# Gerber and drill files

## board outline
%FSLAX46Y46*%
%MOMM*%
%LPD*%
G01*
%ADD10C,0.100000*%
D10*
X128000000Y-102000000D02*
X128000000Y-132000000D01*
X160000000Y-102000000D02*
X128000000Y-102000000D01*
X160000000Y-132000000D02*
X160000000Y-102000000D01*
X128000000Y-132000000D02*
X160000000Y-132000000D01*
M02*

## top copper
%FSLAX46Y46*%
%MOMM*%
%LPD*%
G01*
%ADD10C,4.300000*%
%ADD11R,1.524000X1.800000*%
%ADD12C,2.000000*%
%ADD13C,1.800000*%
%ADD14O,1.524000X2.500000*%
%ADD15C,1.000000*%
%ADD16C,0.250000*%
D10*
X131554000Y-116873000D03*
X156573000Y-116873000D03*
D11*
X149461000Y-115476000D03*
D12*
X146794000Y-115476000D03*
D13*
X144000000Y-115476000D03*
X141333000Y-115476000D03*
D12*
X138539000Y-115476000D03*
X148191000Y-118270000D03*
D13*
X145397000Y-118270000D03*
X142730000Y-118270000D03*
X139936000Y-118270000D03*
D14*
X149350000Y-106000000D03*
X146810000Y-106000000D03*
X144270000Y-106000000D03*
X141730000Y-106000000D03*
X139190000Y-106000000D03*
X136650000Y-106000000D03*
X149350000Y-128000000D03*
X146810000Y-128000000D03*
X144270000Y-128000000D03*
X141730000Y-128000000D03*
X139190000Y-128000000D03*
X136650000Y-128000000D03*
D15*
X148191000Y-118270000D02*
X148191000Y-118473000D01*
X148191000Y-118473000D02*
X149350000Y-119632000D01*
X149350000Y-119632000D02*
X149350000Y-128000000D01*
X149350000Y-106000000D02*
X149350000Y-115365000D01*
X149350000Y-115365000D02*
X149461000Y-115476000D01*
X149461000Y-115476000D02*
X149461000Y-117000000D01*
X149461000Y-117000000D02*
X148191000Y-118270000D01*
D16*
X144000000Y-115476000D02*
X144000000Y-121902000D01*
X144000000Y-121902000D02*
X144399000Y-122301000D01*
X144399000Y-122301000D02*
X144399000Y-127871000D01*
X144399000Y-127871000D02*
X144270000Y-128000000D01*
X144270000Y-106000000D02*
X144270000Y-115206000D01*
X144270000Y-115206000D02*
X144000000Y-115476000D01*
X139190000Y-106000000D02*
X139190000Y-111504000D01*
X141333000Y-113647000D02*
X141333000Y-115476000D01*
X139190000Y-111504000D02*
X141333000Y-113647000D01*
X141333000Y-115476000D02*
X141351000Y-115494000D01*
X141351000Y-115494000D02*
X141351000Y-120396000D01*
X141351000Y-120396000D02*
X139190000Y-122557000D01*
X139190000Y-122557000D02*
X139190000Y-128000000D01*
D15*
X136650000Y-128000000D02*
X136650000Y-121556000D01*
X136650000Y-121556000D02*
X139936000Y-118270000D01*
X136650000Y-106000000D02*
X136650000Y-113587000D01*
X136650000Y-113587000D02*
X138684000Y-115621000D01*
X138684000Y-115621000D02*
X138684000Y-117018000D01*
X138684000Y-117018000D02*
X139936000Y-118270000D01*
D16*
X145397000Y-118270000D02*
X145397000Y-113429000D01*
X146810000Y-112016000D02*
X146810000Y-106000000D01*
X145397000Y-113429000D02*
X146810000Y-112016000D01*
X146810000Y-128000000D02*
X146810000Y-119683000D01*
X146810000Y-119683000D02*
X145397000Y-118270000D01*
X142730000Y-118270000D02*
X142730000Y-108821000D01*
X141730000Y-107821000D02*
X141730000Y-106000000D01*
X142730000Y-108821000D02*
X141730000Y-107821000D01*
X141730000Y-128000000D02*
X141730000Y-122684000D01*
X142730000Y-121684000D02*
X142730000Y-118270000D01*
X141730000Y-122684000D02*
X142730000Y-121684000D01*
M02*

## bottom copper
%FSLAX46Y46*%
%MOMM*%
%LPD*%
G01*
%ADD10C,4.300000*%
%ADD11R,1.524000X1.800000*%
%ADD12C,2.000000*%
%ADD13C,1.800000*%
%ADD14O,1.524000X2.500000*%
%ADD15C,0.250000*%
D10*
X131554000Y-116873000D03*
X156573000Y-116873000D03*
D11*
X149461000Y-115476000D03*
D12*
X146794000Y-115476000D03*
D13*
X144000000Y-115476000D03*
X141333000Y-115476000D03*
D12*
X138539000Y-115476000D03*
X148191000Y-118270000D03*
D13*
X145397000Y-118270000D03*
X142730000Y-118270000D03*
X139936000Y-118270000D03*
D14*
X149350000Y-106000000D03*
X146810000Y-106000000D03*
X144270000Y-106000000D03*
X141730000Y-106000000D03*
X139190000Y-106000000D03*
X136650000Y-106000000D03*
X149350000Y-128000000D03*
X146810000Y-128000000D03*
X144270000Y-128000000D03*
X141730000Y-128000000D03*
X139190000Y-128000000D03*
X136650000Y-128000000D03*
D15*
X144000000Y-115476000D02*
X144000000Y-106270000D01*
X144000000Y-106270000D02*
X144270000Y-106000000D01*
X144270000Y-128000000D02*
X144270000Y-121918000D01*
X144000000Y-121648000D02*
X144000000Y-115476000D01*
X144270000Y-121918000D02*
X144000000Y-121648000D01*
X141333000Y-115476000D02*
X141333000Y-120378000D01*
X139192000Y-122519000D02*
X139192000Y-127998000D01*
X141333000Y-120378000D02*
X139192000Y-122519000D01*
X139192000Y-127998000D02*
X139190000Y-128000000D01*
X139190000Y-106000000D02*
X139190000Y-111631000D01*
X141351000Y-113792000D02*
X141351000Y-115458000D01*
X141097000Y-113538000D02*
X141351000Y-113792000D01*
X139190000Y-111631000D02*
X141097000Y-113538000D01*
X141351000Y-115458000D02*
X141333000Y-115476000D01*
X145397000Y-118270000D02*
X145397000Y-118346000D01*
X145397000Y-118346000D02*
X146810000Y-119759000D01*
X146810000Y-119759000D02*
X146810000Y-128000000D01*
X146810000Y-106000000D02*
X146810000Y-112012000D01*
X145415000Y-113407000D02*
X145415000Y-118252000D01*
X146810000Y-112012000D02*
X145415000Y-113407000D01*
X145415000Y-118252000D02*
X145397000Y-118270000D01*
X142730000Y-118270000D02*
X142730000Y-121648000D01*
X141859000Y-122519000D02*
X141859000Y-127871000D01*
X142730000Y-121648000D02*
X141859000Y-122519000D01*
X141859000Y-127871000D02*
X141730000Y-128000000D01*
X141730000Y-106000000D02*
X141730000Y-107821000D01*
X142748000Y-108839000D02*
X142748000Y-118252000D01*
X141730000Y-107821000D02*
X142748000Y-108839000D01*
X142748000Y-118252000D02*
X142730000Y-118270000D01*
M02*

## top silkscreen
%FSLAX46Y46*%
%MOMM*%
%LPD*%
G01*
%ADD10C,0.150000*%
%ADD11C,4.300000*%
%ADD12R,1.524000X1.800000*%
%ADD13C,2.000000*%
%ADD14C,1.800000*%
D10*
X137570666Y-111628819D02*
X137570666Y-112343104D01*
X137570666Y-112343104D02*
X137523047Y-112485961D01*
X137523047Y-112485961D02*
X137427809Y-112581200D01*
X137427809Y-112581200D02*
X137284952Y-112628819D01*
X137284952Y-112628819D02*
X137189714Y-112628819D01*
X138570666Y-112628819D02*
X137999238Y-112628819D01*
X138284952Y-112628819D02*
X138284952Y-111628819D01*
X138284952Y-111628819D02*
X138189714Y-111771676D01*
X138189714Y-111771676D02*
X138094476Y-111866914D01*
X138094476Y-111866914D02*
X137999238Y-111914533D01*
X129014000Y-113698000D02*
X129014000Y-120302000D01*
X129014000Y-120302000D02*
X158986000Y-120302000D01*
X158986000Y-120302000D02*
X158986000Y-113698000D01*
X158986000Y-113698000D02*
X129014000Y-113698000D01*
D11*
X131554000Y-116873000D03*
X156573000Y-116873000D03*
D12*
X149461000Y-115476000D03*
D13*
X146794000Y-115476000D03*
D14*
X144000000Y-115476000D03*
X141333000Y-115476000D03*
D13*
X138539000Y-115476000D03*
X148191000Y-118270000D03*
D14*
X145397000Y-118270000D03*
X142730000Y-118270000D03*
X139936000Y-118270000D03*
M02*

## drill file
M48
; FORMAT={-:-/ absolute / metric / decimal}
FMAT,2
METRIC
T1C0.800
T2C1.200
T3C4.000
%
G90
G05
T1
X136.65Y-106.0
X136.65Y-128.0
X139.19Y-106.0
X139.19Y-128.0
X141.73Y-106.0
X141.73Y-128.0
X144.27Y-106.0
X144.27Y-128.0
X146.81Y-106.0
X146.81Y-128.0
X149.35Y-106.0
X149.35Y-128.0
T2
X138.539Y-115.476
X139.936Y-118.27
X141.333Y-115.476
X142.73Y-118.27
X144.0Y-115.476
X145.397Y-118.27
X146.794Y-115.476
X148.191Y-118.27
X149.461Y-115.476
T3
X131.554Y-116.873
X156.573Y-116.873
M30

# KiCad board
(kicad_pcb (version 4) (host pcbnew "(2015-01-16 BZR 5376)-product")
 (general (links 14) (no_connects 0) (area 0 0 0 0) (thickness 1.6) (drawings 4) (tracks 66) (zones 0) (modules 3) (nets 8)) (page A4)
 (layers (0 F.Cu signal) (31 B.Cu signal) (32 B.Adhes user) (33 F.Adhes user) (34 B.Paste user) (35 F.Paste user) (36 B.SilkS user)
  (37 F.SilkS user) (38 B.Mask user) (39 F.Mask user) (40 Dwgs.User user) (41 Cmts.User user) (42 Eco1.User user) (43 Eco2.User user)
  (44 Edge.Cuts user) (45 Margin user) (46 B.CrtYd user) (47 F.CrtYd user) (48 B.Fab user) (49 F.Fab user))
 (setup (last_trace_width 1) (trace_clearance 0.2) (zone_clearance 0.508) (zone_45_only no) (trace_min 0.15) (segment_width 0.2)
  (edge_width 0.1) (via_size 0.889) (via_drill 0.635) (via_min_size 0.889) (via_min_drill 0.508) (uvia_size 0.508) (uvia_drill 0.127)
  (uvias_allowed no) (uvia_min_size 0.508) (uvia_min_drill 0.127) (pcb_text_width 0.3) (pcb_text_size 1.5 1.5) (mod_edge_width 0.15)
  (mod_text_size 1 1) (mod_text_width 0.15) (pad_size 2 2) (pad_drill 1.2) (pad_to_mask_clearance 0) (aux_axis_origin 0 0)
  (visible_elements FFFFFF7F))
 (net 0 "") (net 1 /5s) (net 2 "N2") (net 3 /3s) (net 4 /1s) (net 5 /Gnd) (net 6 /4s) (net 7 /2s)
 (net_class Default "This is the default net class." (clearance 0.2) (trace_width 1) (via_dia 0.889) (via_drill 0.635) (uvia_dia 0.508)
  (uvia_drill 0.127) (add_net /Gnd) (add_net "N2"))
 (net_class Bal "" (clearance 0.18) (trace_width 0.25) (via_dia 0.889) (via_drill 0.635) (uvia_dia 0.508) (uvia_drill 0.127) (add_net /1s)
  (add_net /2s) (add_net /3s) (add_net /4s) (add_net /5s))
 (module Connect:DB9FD (layer F.Cu) (at 144 117)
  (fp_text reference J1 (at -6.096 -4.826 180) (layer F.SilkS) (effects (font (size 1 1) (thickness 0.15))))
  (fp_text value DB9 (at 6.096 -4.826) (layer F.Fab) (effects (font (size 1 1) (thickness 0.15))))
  (fp_line (start -14.986 -3.302) (end -14.986 3.302) (layer F.SilkS) (width 0.15))
  (fp_line (start -14.986 3.302) (end 14.986 3.302) (layer F.SilkS) (width 0.15))
  (fp_line (start 14.986 3.302) (end 14.986 -3.302) (layer F.SilkS) (width 0.15))
  (fp_line (start 14.986 -3.302) (end -14.986 -3.302) (layer F.SilkS) (width 0.15))
  (pad "" np_thru_hole circle (at -12.446 -0.127) (size 4.3 4.3) (drill 4) (layers *.Cu *.Mask F.SilkS))
  (pad "" np_thru_hole circle (at 12.573 -0.127) (size 4.3 4.3) (drill 4) (layers *.Cu *.Mask F.SilkS))
  (pad 1 thru_hole rect (at 5.461 -1.524) (size 1.524 1.8) (drill 1.2) (layers *.Cu *.Mask F.SilkS) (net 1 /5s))
  (pad 2 thru_hole circle (at 2.794 -1.524) (size 2 2) (drill 1.2) (layers *.Cu *.Mask F.SilkS) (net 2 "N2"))
  (pad 3 thru_hole circle (at 0 -1.524) (size 1.8 1.8) (drill 1.2) (layers *.Cu *.Mask F.SilkS) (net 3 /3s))
  (pad 4 thru_hole circle (at -2.667 -1.524) (size 1.8 1.8) (drill 1.2) (layers *.Cu *.Mask F.SilkS) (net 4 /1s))
  (pad 5 thru_hole circle (at -5.461 -1.524) (size 2 2) (drill 1.2) (layers *.Cu *.Mask F.SilkS) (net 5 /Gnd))
  (pad 6 thru_hole circle (at 4.191 1.27) (size 2 2) (drill 1.2) (layers *.Cu *.Mask F.SilkS) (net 1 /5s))
  (pad 7 thru_hole circle (at 1.397 1.27) (size 1.8 1.8) (drill 1.2) (layers *.Cu *.Mask F.SilkS) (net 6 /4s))
  (pad 8 thru_hole circle (at -1.27 1.27) (size 1.8 1.8) (drill 1.2) (layers *.Cu *.Mask F.SilkS) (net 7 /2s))
  (pad 9 thru_hole circle (at -4.064 1.27) (size 1.8 1.8) (drill 1.2) (layers *.Cu *.Mask F.SilkS) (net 5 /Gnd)))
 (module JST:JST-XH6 (layer B.Cu) (at 143 106 90)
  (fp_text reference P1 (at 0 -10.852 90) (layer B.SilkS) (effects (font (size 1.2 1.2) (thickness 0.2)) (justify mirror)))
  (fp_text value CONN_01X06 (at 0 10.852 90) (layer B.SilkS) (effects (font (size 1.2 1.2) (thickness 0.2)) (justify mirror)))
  (pad 1 thru_hole oval (at 0 6.35 90) (size 2.5 1.524) (drill 0.8) (layers *.Cu *.Mask B.SilkS) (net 1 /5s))
  (pad 2 thru_hole oval (at 0 3.81 90) (size 2.5 1.524) (drill 0.8) (layers *.Cu *.Mask B.SilkS) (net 6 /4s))
  (pad 3 thru_hole oval (at 0 1.27 90) (size 2.5 1.524) (drill 0.8) (layers *.Cu *.Mask B.SilkS) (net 3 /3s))
  (pad 4 thru_hole oval (at 0 -1.27 90) (size 2.5 1.524) (drill 0.8) (layers *.Cu *.Mask B.SilkS) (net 7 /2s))
  (pad 5 thru_hole oval (at 0 -3.81 90) (size 2.5 1.524) (drill 0.8) (layers *.Cu *.Mask B.SilkS) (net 4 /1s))
  (pad 6 thru_hole oval (at 0 -6.35 90) (size 2.5 1.524) (drill 0.8) (layers *.Cu *.Mask B.SilkS) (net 5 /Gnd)))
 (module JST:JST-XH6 (layer B.Cu) (at 143 128 90)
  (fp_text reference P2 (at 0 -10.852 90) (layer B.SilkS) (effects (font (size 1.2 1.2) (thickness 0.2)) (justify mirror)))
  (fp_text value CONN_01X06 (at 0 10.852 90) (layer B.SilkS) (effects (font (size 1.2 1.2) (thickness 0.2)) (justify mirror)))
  (pad 1 thru_hole oval (at 0 6.35 90) (size 2.5 1.524) (drill 0.8) (layers *.Cu *.Mask B.SilkS) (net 1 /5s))
  (pad 2 thru_hole oval (at 0 3.81 90) (size 2.5 1.524) (drill 0.8) (layers *.Cu *.Mask B.SilkS) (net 6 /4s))
  (pad 3 thru_hole oval (at 0 1.27 90) (size 2.5 1.524) (drill 0.8) (layers *.Cu *.Mask B.SilkS) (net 3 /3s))
  (pad 4 thru_hole oval (at 0 -1.27 90) (size 2.5 1.524) (drill 0.8) (layers *.Cu *.Mask B.SilkS) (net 7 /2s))
  (pad 5 thru_hole oval (at 0 -3.81 90) (size 2.5 1.524) (drill 0.8) (layers *.Cu *.Mask B.SilkS) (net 4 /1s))
  (pad 6 thru_hole oval (at 0 -6.35 90) (size 2.5 1.524) (drill 0.8) (layers *.Cu *.Mask B.SilkS) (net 5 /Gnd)))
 (gr_line (start 128 102) (end 128 132) (angle 90) (layer Edge.Cuts) (width 0.1))
 (gr_line (start 160 102) (end 128 102) (angle 90) (layer Edge.Cuts) (width 0.1))
 (gr_line (start 160 132) (end 160 102) (angle 90) (layer Edge.Cuts) (width 0.1))
 (gr_line (start 128 132) (end 160 132) (angle 90) (layer Edge.Cuts) (width 0.1))
 (segment (start 148.191 118.27) (end 148.191 118.473) (width 1) (layer F.Cu) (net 1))
 (segment (start 148.191 118.473) (end 149.35 119.632) (width 1) (layer F.Cu) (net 1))
 (segment (start 149.35 119.632) (end 149.35 128) (width 1) (layer F.Cu) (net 1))
 (segment (start 149.35 106) (end 149.35 115.365) (width 1) (layer F.Cu) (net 1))
 (segment (start 149.35 115.365) (end 149.461 115.476) (width 1) (layer F.Cu) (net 1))
 (segment (start 149.461 115.476) (end 149.461 117) (width 1) (layer F.Cu) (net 1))
 (segment (start 149.461 117) (end 148.191 118.27) (width 1) (layer F.Cu) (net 1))
 (segment (start 144 115.476) (end 144 106.27) (width 0.25) (layer B.Cu) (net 3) (status C00000))
 (segment (start 144 106.27) (end 144.27 106) (width 0.25) (layer B.Cu) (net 3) (status C00000))
 (segment (start 144.27 128) (end 144.27 121.918) (width 0.25) (layer B.Cu) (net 3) (status 400000))
 (segment (start 144 121.648) (end 144 115.476) (width 0.25) (layer B.Cu) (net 3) (status 800000))
 (segment (start 144.27 121.918) (end 144 121.648) (width 0.25) (layer B.Cu) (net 3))
 (segment (start 144 115.476) (end 144 121.902) (width 0.25) (layer F.Cu) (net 3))
 (segment (start 144 121.902) (end 144.399 122.301) (width 0.25) (layer F.Cu) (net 3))
 (segment (start 144.399 122.301) (end 144.399 127.871) (width 0.25) (layer F.Cu) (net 3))
 (segment (start 144.399 127.871) (end 144.27 128) (width 0.25) (layer F.Cu) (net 3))
 (segment (start 144.27 106) (end 144.27 115.206) (width 0.25) (layer F.Cu) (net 3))
 (segment (start 144.27 115.206) (end 144 115.476) (width 0.25) (layer F.Cu) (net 3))
 (segment (start 141.333 115.476) (end 141.333 120.378) (width 0.25) (layer B.Cu) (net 4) (status 400000))
 (segment (start 139.192 122.519) (end 139.192 127.998) (width 0.25) (layer B.Cu) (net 4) (status 800000))
 (segment (start 141.333 120.378) (end 139.192 122.519) (width 0.25) (layer B.Cu) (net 4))
 (segment (start 139.192 127.998) (end 139.19 128) (width 0.25) (layer B.Cu) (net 4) (status C00000))
 (segment (start 139.19 106) (end 139.19 111.631) (width 0.25) (layer B.Cu) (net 4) (status 400000))
 (segment (start 141.351 113.792) (end 141.351 115.458) (width 0.25) (layer B.Cu) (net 4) (status 800000))
 (segment (start 141.097 113.538) (end 141.351 113.792) (width 0.25) (layer B.Cu) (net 4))
 (segment (start 139.19 111.631) (end 141.097 113.538) (width 0.25) (layer B.Cu) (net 4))
 (segment (start 141.351 115.458) (end 141.333 115.476) (width 0.25) (layer B.Cu) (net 4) (status C00000))
 (segment (start 139.19 106) (end 139.19 111.504) (width 0.25) (layer F.Cu) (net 4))
 (segment (start 141.333 113.647) (end 141.333 115.476) (width 0.25) (layer F.Cu) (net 4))
 (segment (start 139.19 111.504) (end 141.333 113.647) (width 0.25) (layer F.Cu) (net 4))
 (segment (start 141.333 115.476) (end 141.351 115.494) (width 0.25) (layer F.Cu) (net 4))
 (segment (start 141.351 115.494) (end 141.351 120.396) (width 0.25) (layer F.Cu) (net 4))
 (segment (start 141.351 120.396) (end 139.19 122.557) (width 0.25) (layer F.Cu) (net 4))
 (segment (start 139.19 122.557) (end 139.19 128) (width 0.25) (layer F.Cu) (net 4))
 (segment (start 136.65 128) (end 136.65 121.556) (width 1) (layer F.Cu) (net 5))
 (segment (start 136.65 121.556) (end 139.936 118.27) (width 1) (layer F.Cu) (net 5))
 (segment (start 136.65 106) (end 136.65 113.587) (width 1) (layer F.Cu) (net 5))
 (segment (start 136.65 113.587) (end 138.684 115.621) (width 1) (layer F.Cu) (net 5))
 (segment (start 138.684 115.621) (end 138.684 117.018) (width 1) (layer F.Cu) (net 5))
 (segment (start 138.684 117.018) (end 139.936 118.27) (width 1) (layer F.Cu) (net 5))
 (segment (start 145.397 118.27) (end 145.397 118.346) (width 0.25) (layer B.Cu) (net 6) (status C00000))
 (segment (start 145.397 118.346) (end 146.81 119.759) (width 0.25) (layer B.Cu) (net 6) (status 400000))
 (segment (start 146.81 119.759) (end 146.81 128) (width 0.25) (layer B.Cu) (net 6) (status 800000))
 (segment (start 146.81 106) (end 146.81 112.012) (width 0.25) (layer B.Cu) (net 6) (status 400000))
 (segment (start 145.415 113.407) (end 145.415 118.252) (width 0.25) (layer B.Cu) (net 6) (status 800000))
 (segment (start 146.81 112.012) (end 145.415 113.407) (width 0.25) (layer B.Cu) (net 6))
 (segment (start 145.415 118.252) (end 145.397 118.27) (width 0.25) (layer B.Cu) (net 6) (status C00000))
 (segment (start 145.397 118.27) (end 145.397 113.429) (width 0.25) (layer F.Cu) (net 6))
 (segment (start 146.81 112.016) (end 146.81 106) (width 0.25) (layer F.Cu) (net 6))
 (segment (start 145.397 113.429) (end 146.81 112.016) (width 0.25) (layer F.Cu) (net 6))
 (segment (start 146.81 128) (end 146.81 119.683) (width 0.25) (layer F.Cu) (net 6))
 (segment (start 146.81 119.683) (end 145.397 118.27) (width 0.25) (layer F.Cu) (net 6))
 (segment (start 142.73 118.27) (end 142.73 121.648) (width 0.25) (layer B.Cu) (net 7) (status 400000))
 (segment (start 141.859 122.519) (end 141.859 127.871) (width 0.25) (layer B.Cu) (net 7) (status 800000))
 (segment (start 142.73 121.648) (end 141.859 122.519) (width 0.25) (layer B.Cu) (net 7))
 (segment (start 141.859 127.871) (end 141.73 128) (width 0.25) (layer B.Cu) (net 7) (status C00000))
 (segment (start 141.73 106) (end 141.73 107.821) (width 0.25) (layer B.Cu) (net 7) (status 400000))
 (segment (start 142.748 108.839) (end 142.748 118.252) (width 0.25) (layer B.Cu) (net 7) (status 800000))
 (segment (start 141.73 107.821) (end 142.748 108.839) (width 0.25) (layer B.Cu) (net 7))
 (segment (start 142.748 118.252) (end 142.73 118.27) (width 0.25) (layer B.Cu) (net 7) (status C00000))
 (segment (start 142.73 118.27) (end 142.73 108.821) (width 0.25) (layer F.Cu) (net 7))
 (segment (start 141.73 107.821) (end 141.73 106) (width 0.25) (layer F.Cu) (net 7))
 (segment (start 142.73 108.821) (end 141.73 107.821) (width 0.25) (layer F.Cu) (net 7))
 (segment (start 141.73 128) (end 141.73 122.684) (width 0.25) (layer F.Cu) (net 7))
 (segment (start 142.73 121.684) (end 142.73 118.27) (width 0.25) (layer F.Cu) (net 7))
 (segment (start 141.73 122.684) (end 142.73 121.684) (width 0.25) (layer F.Cu) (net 7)))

